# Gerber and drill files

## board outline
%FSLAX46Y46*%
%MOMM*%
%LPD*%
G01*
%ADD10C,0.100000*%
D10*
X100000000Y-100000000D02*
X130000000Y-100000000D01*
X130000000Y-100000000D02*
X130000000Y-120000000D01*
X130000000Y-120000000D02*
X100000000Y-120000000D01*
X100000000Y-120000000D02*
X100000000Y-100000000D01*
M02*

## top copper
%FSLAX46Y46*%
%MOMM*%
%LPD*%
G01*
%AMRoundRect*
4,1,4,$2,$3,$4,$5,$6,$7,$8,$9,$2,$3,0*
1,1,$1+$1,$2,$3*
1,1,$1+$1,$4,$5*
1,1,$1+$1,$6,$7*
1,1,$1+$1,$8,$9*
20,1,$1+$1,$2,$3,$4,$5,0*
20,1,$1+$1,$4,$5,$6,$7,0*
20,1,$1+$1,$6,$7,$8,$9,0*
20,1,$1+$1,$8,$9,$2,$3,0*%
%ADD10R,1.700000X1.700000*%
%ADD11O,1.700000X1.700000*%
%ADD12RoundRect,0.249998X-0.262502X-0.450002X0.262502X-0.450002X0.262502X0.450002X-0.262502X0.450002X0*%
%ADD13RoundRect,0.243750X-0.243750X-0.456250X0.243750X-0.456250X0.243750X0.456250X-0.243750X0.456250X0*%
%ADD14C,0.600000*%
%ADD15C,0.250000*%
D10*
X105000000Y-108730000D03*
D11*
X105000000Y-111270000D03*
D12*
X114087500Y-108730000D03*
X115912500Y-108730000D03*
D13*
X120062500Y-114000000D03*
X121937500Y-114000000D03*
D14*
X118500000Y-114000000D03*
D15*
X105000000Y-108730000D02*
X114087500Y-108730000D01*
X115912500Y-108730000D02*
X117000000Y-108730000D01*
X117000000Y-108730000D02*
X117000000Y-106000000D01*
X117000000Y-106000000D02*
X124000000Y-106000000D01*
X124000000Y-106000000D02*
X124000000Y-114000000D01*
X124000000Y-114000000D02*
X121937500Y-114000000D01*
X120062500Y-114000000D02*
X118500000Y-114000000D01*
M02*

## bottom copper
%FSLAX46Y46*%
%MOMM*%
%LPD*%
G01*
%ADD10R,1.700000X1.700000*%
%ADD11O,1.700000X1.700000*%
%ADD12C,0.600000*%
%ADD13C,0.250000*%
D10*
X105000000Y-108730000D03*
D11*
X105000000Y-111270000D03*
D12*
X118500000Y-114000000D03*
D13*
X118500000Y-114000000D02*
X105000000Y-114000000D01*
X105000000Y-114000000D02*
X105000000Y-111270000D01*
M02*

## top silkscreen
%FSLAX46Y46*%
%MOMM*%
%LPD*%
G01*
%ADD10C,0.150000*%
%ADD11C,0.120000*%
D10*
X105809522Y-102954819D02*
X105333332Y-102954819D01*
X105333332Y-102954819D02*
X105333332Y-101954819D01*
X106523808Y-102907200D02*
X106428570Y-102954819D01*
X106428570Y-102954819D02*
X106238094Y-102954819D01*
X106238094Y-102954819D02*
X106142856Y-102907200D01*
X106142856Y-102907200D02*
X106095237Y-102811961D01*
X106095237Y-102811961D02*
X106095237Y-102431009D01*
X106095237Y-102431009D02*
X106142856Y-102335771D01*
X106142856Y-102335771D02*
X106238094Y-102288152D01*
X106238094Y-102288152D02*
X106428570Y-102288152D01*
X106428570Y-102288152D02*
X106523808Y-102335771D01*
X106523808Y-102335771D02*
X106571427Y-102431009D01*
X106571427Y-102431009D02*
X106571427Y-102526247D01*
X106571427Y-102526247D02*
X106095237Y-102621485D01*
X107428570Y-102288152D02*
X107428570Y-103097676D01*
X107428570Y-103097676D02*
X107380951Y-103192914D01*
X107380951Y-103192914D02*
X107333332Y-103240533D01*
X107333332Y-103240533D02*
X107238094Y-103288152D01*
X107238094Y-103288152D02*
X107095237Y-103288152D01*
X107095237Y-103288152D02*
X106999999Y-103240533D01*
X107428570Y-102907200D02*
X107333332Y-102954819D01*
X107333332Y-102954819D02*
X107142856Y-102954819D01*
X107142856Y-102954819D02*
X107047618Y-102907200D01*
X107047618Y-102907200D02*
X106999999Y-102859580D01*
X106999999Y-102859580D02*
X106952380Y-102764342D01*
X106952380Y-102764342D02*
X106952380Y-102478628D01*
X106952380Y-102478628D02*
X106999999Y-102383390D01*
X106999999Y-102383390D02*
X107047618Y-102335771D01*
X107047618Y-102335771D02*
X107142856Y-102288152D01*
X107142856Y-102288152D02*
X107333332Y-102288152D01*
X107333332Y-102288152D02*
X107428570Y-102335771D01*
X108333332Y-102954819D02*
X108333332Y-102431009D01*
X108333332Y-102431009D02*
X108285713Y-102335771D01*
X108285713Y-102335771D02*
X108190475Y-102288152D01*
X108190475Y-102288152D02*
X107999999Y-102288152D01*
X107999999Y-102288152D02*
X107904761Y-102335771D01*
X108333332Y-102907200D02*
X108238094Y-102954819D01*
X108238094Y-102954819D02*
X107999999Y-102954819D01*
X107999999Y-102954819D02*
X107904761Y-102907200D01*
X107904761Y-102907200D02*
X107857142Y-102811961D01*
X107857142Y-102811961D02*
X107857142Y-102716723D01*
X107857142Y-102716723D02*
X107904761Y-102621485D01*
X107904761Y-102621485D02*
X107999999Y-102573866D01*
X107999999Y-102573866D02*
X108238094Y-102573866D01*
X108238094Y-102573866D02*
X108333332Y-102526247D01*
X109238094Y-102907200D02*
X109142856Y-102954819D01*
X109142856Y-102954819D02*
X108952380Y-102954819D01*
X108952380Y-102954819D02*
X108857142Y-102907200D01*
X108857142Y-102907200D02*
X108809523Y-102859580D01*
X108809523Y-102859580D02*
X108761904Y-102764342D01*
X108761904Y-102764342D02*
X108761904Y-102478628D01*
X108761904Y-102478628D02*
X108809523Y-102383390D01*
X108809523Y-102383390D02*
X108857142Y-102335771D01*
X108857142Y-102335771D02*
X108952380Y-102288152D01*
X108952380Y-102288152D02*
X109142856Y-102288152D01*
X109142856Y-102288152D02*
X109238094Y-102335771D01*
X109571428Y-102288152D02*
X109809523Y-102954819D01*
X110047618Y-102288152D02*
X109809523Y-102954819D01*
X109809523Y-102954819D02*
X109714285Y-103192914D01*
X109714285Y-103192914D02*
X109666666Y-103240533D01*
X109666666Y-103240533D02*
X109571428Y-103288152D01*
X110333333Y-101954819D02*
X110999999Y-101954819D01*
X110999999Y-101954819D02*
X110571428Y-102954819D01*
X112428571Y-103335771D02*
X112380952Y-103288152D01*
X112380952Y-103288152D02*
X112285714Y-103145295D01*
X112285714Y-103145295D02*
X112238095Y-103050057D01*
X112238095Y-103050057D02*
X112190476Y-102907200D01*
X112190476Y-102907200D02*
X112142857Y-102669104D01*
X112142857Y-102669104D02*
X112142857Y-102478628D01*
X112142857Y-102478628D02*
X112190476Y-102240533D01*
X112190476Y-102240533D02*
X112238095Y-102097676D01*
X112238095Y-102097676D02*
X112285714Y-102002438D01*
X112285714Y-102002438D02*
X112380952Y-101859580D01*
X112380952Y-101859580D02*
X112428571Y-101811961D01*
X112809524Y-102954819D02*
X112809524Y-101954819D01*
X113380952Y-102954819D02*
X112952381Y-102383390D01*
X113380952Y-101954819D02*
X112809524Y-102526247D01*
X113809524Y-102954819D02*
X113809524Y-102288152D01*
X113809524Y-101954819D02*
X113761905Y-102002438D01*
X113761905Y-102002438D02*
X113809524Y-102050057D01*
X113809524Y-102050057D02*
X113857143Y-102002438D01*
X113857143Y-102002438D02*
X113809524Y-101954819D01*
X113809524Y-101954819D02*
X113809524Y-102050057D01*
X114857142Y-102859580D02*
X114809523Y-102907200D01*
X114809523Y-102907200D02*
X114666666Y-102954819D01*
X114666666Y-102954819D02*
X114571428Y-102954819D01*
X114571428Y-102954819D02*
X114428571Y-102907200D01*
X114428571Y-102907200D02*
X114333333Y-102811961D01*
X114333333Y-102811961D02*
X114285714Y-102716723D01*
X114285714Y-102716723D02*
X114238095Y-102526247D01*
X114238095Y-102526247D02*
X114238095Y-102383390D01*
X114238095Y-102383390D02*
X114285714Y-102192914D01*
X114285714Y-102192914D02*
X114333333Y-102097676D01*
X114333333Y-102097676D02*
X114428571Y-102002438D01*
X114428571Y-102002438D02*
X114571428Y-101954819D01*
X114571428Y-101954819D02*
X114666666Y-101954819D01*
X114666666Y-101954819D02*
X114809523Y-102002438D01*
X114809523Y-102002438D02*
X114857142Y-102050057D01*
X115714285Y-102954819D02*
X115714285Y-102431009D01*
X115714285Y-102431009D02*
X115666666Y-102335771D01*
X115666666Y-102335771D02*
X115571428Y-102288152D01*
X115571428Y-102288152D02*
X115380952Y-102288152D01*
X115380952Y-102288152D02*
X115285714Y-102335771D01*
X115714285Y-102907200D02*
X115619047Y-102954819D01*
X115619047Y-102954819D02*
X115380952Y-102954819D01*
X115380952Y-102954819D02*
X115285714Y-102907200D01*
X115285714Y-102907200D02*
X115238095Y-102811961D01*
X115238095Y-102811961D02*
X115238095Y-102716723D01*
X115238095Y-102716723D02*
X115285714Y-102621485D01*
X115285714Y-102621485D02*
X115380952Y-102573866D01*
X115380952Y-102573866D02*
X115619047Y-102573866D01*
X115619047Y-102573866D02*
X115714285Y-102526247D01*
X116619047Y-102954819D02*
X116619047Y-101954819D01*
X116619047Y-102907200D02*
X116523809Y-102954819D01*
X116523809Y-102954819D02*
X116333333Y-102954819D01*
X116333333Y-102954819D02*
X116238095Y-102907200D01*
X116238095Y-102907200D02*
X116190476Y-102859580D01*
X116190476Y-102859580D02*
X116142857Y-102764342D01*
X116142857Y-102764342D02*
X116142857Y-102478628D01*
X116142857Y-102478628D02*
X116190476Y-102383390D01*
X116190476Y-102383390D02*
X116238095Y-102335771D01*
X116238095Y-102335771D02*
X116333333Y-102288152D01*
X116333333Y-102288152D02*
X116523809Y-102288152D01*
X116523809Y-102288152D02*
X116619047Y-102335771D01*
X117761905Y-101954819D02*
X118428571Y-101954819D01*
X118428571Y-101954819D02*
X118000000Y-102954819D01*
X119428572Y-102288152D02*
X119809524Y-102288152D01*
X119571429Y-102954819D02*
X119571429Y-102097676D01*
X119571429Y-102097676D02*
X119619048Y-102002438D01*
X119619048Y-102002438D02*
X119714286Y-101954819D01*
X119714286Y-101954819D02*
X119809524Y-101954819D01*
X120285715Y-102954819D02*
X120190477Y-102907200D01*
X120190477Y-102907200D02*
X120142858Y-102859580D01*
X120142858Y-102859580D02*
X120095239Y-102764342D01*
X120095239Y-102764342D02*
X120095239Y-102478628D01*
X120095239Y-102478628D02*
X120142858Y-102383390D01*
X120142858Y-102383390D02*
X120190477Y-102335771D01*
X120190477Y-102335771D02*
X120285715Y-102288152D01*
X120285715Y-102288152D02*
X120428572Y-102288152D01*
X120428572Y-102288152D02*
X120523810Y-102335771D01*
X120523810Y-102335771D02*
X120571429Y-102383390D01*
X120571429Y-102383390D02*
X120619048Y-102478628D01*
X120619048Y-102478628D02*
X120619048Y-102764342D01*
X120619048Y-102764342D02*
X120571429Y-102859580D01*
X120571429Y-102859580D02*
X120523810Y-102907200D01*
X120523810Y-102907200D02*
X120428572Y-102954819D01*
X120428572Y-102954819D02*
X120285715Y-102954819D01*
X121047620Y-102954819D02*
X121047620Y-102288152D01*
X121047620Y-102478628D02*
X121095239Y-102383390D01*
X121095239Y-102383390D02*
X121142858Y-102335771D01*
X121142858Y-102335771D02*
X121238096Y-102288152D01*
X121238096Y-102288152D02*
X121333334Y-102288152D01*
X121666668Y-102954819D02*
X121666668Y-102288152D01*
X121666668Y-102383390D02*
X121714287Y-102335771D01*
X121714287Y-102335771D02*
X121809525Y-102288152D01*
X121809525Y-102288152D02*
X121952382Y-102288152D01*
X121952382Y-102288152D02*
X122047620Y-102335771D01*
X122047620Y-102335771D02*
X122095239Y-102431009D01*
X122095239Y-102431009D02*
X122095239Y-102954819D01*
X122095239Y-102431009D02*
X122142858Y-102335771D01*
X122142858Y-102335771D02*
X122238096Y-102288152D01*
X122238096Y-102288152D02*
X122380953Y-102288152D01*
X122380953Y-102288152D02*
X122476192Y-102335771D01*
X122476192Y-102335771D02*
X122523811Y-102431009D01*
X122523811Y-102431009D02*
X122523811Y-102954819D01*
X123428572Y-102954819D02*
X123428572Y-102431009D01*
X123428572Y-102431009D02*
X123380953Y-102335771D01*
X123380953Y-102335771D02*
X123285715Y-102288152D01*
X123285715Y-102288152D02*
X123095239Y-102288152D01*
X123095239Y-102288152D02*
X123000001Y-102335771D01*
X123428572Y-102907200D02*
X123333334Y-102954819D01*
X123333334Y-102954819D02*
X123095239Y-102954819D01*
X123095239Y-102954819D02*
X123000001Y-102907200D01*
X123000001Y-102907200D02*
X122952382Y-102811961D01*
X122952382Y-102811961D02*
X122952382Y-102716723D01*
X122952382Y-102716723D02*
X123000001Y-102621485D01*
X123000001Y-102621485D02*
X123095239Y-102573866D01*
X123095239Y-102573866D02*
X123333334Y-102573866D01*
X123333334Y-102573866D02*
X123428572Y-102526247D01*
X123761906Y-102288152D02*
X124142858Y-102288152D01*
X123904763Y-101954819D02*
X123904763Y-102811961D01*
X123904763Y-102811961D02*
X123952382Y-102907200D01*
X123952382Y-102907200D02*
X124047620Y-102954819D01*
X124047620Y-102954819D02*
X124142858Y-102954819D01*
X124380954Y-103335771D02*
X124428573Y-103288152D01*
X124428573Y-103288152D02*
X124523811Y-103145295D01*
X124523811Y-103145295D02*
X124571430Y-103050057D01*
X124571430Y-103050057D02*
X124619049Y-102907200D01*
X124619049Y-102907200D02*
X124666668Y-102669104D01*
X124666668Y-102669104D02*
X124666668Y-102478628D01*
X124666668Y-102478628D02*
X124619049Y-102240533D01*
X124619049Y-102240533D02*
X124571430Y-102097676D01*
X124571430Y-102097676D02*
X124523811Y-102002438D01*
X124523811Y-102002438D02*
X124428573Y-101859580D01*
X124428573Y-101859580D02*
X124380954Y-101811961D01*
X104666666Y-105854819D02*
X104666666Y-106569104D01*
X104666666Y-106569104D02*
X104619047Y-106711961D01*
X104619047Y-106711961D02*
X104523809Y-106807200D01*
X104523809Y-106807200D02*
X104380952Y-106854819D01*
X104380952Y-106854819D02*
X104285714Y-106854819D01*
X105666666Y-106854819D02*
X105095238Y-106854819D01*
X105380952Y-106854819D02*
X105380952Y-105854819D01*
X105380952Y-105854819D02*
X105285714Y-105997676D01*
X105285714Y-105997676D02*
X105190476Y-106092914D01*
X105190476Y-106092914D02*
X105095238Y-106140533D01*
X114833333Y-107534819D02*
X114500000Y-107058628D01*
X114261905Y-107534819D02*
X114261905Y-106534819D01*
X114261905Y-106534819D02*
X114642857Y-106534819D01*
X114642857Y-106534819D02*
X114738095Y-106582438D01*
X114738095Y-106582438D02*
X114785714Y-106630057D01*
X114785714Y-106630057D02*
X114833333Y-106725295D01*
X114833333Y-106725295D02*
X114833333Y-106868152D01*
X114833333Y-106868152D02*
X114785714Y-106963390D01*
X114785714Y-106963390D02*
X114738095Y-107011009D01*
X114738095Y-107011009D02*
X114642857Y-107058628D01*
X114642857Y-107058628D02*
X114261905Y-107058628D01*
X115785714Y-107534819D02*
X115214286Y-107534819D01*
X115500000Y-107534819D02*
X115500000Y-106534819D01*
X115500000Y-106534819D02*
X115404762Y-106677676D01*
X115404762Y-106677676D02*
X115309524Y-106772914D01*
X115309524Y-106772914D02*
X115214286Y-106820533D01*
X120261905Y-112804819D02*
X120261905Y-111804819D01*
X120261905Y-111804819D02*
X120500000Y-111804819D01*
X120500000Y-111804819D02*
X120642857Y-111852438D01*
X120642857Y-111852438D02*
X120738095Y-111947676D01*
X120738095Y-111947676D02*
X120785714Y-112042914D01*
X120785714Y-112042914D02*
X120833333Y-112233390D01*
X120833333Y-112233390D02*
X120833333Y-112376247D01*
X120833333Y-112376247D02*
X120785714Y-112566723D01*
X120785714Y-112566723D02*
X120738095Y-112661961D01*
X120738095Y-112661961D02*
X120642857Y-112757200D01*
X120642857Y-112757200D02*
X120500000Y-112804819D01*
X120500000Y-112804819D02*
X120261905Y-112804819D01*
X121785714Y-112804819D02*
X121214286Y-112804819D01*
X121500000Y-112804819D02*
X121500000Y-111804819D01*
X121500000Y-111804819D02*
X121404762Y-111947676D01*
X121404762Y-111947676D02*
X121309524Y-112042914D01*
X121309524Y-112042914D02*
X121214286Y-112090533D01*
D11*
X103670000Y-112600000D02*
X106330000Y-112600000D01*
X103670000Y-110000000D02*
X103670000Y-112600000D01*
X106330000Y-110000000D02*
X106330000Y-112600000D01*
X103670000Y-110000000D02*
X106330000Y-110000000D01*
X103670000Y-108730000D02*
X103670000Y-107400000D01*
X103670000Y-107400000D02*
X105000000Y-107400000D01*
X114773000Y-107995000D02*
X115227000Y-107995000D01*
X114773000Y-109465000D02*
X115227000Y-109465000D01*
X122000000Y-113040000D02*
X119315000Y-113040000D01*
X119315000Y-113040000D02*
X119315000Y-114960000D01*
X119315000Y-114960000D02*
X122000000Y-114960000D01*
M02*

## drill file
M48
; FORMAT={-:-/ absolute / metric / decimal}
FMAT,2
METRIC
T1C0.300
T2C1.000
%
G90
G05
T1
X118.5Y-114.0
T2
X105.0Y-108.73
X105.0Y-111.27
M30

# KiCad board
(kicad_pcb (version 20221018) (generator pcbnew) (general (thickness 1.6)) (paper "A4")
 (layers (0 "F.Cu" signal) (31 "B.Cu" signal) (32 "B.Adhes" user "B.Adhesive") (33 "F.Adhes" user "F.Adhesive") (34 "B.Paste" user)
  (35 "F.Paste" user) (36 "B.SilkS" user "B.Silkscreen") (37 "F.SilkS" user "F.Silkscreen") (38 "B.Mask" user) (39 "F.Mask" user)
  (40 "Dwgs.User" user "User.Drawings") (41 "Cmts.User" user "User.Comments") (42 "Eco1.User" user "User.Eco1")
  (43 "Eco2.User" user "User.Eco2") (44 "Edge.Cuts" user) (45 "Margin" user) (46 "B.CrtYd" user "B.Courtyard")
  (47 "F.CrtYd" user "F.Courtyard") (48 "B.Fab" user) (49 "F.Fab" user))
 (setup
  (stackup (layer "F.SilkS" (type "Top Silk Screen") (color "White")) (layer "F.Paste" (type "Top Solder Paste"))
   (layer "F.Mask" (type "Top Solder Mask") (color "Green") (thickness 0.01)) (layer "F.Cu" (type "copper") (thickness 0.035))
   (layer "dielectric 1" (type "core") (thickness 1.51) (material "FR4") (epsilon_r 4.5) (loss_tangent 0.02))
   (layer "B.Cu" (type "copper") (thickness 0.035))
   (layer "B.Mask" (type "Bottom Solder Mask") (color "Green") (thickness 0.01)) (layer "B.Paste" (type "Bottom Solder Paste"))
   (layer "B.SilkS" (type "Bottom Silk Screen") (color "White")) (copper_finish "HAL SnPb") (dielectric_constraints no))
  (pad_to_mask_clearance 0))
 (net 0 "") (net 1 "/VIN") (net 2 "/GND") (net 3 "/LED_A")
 (gr_line (start 100 100) (end 130 100) (stroke (width 0.1) (type default)) (layer "Edge.Cuts"))
 (gr_line (start 130 100) (end 130 120) (stroke (width 0.1) (type default)) (layer "Edge.Cuts"))
 (gr_line (start 130 120) (end 100 120) (stroke (width 0.1) (type default)) (layer "Edge.Cuts"))
 (gr_line (start 100 120) (end 100 100) (stroke (width 0.1) (type default)) (layer "Edge.Cuts"))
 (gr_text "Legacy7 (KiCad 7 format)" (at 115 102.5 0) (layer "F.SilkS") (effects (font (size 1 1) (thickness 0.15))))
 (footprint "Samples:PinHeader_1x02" (layer "F.Cu") (at 105 108.73)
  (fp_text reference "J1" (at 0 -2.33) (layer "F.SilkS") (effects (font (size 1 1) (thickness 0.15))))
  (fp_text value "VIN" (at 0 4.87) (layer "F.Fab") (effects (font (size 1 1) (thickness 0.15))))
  (fp_line (start -1.33 3.87) (end 1.33 3.87) (stroke (width 0.12) (type solid)) (layer "F.SilkS"))
  (fp_line (start -1.33 1.27) (end -1.33 3.87) (stroke (width 0.12) (type solid)) (layer "F.SilkS"))
  (fp_line (start 1.33 1.27) (end 1.33 3.87) (stroke (width 0.12) (type solid)) (layer "F.SilkS"))
  (fp_line (start -1.33 1.27) (end 1.33 1.27) (stroke (width 0.12) (type solid)) (layer "F.SilkS"))
  (fp_line (start -1.33 0) (end -1.33 -1.33) (stroke (width 0.12) (type solid)) (layer "F.SilkS"))
  (fp_line (start -1.33 -1.33) (end 0 -1.33) (stroke (width 0.12) (type solid)) (layer "F.SilkS"))
  (pad "1" thru_hole rect (at 0 0) (size 1.7 1.7) (drill 1) (layers "*.Cu" "*.Mask") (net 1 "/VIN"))
  (pad "2" thru_hole oval (at 0 2.54) (size 1.7 1.7) (drill 1) (layers "*.Cu" "*.Mask") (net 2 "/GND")))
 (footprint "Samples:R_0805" (layer "F.Cu") (at 115 108.73)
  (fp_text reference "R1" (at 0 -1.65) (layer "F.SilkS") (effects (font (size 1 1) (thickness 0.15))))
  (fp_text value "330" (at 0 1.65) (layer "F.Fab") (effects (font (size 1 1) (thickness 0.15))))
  (fp_line (start -0.227 -0.735) (end 0.227 -0.735) (stroke (width 0.12) (type solid)) (layer "F.SilkS"))
  (fp_line (start -0.227 0.735) (end 0.227 0.735) (stroke (width 0.12) (type solid)) (layer "F.SilkS"))
  (pad "1" smd roundrect (at -0.9125 0) (size 1.025 1.4) (layers "F.Cu" "F.Paste" "F.Mask") (roundrect_rratio 0.2439) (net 1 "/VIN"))
  (pad "2" smd roundrect (at 0.9125 0) (size 1.025 1.4) (layers "F.Cu" "F.Paste" "F.Mask") (roundrect_rratio 0.2439) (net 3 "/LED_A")))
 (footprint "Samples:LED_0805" (layer "F.Cu") (at 121 114)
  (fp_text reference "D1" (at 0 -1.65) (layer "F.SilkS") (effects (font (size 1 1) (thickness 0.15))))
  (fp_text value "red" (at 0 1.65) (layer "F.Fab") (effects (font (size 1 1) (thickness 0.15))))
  (fp_line (start 1 -0.96) (end -1.685 -0.96) (stroke (width 0.12) (type solid)) (layer "F.SilkS"))
  (fp_line (start -1.685 -0.96) (end -1.685 0.96) (stroke (width 0.12) (type solid)) (layer "F.SilkS"))
  (fp_line (start -1.685 0.96) (end 1 0.96) (stroke (width 0.12) (type solid)) (layer "F.SilkS"))
  (pad "1" smd roundrect (at -0.9375 0) (size 0.975 1.4) (layers "F.Cu" "F.Paste" "F.Mask") (roundrect_rratio 0.25) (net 2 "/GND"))
  (pad "2" smd roundrect (at 0.9375 0) (size 0.975 1.4) (layers "F.Cu" "F.Paste" "F.Mask") (roundrect_rratio 0.25) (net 3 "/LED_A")))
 (segment (start 105 108.73) (end 114.0875 108.73) (width 0.25) (layer "F.Cu") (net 1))
 (segment (start 115.9125 108.73) (end 117 108.73) (width 0.25) (layer "F.Cu") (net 3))
 (segment (start 117 108.73) (end 117 106) (width 0.25) (layer "F.Cu") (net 3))
 (segment (start 117 106) (end 124 106) (width 0.25) (layer "F.Cu") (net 3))
 (segment (start 124 106) (end 124 114) (width 0.25) (layer "F.Cu") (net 3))
 (segment (start 124 114) (end 121.9375 114) (width 0.25) (layer "F.Cu") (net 3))
 (segment (start 120.0625 114) (end 118.5 114) (width 0.25) (layer "F.Cu") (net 2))
 (segment (start 118.5 114) (end 105 114) (width 0.25) (layer "B.Cu") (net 2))
 (segment (start 105 114) (end 105 111.27) (width 0.25) (layer "B.Cu") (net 2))
 (via (at 118.5 114) (size 0.6) (drill 0.3) (layers "F.Cu" "B.Cu") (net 2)))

